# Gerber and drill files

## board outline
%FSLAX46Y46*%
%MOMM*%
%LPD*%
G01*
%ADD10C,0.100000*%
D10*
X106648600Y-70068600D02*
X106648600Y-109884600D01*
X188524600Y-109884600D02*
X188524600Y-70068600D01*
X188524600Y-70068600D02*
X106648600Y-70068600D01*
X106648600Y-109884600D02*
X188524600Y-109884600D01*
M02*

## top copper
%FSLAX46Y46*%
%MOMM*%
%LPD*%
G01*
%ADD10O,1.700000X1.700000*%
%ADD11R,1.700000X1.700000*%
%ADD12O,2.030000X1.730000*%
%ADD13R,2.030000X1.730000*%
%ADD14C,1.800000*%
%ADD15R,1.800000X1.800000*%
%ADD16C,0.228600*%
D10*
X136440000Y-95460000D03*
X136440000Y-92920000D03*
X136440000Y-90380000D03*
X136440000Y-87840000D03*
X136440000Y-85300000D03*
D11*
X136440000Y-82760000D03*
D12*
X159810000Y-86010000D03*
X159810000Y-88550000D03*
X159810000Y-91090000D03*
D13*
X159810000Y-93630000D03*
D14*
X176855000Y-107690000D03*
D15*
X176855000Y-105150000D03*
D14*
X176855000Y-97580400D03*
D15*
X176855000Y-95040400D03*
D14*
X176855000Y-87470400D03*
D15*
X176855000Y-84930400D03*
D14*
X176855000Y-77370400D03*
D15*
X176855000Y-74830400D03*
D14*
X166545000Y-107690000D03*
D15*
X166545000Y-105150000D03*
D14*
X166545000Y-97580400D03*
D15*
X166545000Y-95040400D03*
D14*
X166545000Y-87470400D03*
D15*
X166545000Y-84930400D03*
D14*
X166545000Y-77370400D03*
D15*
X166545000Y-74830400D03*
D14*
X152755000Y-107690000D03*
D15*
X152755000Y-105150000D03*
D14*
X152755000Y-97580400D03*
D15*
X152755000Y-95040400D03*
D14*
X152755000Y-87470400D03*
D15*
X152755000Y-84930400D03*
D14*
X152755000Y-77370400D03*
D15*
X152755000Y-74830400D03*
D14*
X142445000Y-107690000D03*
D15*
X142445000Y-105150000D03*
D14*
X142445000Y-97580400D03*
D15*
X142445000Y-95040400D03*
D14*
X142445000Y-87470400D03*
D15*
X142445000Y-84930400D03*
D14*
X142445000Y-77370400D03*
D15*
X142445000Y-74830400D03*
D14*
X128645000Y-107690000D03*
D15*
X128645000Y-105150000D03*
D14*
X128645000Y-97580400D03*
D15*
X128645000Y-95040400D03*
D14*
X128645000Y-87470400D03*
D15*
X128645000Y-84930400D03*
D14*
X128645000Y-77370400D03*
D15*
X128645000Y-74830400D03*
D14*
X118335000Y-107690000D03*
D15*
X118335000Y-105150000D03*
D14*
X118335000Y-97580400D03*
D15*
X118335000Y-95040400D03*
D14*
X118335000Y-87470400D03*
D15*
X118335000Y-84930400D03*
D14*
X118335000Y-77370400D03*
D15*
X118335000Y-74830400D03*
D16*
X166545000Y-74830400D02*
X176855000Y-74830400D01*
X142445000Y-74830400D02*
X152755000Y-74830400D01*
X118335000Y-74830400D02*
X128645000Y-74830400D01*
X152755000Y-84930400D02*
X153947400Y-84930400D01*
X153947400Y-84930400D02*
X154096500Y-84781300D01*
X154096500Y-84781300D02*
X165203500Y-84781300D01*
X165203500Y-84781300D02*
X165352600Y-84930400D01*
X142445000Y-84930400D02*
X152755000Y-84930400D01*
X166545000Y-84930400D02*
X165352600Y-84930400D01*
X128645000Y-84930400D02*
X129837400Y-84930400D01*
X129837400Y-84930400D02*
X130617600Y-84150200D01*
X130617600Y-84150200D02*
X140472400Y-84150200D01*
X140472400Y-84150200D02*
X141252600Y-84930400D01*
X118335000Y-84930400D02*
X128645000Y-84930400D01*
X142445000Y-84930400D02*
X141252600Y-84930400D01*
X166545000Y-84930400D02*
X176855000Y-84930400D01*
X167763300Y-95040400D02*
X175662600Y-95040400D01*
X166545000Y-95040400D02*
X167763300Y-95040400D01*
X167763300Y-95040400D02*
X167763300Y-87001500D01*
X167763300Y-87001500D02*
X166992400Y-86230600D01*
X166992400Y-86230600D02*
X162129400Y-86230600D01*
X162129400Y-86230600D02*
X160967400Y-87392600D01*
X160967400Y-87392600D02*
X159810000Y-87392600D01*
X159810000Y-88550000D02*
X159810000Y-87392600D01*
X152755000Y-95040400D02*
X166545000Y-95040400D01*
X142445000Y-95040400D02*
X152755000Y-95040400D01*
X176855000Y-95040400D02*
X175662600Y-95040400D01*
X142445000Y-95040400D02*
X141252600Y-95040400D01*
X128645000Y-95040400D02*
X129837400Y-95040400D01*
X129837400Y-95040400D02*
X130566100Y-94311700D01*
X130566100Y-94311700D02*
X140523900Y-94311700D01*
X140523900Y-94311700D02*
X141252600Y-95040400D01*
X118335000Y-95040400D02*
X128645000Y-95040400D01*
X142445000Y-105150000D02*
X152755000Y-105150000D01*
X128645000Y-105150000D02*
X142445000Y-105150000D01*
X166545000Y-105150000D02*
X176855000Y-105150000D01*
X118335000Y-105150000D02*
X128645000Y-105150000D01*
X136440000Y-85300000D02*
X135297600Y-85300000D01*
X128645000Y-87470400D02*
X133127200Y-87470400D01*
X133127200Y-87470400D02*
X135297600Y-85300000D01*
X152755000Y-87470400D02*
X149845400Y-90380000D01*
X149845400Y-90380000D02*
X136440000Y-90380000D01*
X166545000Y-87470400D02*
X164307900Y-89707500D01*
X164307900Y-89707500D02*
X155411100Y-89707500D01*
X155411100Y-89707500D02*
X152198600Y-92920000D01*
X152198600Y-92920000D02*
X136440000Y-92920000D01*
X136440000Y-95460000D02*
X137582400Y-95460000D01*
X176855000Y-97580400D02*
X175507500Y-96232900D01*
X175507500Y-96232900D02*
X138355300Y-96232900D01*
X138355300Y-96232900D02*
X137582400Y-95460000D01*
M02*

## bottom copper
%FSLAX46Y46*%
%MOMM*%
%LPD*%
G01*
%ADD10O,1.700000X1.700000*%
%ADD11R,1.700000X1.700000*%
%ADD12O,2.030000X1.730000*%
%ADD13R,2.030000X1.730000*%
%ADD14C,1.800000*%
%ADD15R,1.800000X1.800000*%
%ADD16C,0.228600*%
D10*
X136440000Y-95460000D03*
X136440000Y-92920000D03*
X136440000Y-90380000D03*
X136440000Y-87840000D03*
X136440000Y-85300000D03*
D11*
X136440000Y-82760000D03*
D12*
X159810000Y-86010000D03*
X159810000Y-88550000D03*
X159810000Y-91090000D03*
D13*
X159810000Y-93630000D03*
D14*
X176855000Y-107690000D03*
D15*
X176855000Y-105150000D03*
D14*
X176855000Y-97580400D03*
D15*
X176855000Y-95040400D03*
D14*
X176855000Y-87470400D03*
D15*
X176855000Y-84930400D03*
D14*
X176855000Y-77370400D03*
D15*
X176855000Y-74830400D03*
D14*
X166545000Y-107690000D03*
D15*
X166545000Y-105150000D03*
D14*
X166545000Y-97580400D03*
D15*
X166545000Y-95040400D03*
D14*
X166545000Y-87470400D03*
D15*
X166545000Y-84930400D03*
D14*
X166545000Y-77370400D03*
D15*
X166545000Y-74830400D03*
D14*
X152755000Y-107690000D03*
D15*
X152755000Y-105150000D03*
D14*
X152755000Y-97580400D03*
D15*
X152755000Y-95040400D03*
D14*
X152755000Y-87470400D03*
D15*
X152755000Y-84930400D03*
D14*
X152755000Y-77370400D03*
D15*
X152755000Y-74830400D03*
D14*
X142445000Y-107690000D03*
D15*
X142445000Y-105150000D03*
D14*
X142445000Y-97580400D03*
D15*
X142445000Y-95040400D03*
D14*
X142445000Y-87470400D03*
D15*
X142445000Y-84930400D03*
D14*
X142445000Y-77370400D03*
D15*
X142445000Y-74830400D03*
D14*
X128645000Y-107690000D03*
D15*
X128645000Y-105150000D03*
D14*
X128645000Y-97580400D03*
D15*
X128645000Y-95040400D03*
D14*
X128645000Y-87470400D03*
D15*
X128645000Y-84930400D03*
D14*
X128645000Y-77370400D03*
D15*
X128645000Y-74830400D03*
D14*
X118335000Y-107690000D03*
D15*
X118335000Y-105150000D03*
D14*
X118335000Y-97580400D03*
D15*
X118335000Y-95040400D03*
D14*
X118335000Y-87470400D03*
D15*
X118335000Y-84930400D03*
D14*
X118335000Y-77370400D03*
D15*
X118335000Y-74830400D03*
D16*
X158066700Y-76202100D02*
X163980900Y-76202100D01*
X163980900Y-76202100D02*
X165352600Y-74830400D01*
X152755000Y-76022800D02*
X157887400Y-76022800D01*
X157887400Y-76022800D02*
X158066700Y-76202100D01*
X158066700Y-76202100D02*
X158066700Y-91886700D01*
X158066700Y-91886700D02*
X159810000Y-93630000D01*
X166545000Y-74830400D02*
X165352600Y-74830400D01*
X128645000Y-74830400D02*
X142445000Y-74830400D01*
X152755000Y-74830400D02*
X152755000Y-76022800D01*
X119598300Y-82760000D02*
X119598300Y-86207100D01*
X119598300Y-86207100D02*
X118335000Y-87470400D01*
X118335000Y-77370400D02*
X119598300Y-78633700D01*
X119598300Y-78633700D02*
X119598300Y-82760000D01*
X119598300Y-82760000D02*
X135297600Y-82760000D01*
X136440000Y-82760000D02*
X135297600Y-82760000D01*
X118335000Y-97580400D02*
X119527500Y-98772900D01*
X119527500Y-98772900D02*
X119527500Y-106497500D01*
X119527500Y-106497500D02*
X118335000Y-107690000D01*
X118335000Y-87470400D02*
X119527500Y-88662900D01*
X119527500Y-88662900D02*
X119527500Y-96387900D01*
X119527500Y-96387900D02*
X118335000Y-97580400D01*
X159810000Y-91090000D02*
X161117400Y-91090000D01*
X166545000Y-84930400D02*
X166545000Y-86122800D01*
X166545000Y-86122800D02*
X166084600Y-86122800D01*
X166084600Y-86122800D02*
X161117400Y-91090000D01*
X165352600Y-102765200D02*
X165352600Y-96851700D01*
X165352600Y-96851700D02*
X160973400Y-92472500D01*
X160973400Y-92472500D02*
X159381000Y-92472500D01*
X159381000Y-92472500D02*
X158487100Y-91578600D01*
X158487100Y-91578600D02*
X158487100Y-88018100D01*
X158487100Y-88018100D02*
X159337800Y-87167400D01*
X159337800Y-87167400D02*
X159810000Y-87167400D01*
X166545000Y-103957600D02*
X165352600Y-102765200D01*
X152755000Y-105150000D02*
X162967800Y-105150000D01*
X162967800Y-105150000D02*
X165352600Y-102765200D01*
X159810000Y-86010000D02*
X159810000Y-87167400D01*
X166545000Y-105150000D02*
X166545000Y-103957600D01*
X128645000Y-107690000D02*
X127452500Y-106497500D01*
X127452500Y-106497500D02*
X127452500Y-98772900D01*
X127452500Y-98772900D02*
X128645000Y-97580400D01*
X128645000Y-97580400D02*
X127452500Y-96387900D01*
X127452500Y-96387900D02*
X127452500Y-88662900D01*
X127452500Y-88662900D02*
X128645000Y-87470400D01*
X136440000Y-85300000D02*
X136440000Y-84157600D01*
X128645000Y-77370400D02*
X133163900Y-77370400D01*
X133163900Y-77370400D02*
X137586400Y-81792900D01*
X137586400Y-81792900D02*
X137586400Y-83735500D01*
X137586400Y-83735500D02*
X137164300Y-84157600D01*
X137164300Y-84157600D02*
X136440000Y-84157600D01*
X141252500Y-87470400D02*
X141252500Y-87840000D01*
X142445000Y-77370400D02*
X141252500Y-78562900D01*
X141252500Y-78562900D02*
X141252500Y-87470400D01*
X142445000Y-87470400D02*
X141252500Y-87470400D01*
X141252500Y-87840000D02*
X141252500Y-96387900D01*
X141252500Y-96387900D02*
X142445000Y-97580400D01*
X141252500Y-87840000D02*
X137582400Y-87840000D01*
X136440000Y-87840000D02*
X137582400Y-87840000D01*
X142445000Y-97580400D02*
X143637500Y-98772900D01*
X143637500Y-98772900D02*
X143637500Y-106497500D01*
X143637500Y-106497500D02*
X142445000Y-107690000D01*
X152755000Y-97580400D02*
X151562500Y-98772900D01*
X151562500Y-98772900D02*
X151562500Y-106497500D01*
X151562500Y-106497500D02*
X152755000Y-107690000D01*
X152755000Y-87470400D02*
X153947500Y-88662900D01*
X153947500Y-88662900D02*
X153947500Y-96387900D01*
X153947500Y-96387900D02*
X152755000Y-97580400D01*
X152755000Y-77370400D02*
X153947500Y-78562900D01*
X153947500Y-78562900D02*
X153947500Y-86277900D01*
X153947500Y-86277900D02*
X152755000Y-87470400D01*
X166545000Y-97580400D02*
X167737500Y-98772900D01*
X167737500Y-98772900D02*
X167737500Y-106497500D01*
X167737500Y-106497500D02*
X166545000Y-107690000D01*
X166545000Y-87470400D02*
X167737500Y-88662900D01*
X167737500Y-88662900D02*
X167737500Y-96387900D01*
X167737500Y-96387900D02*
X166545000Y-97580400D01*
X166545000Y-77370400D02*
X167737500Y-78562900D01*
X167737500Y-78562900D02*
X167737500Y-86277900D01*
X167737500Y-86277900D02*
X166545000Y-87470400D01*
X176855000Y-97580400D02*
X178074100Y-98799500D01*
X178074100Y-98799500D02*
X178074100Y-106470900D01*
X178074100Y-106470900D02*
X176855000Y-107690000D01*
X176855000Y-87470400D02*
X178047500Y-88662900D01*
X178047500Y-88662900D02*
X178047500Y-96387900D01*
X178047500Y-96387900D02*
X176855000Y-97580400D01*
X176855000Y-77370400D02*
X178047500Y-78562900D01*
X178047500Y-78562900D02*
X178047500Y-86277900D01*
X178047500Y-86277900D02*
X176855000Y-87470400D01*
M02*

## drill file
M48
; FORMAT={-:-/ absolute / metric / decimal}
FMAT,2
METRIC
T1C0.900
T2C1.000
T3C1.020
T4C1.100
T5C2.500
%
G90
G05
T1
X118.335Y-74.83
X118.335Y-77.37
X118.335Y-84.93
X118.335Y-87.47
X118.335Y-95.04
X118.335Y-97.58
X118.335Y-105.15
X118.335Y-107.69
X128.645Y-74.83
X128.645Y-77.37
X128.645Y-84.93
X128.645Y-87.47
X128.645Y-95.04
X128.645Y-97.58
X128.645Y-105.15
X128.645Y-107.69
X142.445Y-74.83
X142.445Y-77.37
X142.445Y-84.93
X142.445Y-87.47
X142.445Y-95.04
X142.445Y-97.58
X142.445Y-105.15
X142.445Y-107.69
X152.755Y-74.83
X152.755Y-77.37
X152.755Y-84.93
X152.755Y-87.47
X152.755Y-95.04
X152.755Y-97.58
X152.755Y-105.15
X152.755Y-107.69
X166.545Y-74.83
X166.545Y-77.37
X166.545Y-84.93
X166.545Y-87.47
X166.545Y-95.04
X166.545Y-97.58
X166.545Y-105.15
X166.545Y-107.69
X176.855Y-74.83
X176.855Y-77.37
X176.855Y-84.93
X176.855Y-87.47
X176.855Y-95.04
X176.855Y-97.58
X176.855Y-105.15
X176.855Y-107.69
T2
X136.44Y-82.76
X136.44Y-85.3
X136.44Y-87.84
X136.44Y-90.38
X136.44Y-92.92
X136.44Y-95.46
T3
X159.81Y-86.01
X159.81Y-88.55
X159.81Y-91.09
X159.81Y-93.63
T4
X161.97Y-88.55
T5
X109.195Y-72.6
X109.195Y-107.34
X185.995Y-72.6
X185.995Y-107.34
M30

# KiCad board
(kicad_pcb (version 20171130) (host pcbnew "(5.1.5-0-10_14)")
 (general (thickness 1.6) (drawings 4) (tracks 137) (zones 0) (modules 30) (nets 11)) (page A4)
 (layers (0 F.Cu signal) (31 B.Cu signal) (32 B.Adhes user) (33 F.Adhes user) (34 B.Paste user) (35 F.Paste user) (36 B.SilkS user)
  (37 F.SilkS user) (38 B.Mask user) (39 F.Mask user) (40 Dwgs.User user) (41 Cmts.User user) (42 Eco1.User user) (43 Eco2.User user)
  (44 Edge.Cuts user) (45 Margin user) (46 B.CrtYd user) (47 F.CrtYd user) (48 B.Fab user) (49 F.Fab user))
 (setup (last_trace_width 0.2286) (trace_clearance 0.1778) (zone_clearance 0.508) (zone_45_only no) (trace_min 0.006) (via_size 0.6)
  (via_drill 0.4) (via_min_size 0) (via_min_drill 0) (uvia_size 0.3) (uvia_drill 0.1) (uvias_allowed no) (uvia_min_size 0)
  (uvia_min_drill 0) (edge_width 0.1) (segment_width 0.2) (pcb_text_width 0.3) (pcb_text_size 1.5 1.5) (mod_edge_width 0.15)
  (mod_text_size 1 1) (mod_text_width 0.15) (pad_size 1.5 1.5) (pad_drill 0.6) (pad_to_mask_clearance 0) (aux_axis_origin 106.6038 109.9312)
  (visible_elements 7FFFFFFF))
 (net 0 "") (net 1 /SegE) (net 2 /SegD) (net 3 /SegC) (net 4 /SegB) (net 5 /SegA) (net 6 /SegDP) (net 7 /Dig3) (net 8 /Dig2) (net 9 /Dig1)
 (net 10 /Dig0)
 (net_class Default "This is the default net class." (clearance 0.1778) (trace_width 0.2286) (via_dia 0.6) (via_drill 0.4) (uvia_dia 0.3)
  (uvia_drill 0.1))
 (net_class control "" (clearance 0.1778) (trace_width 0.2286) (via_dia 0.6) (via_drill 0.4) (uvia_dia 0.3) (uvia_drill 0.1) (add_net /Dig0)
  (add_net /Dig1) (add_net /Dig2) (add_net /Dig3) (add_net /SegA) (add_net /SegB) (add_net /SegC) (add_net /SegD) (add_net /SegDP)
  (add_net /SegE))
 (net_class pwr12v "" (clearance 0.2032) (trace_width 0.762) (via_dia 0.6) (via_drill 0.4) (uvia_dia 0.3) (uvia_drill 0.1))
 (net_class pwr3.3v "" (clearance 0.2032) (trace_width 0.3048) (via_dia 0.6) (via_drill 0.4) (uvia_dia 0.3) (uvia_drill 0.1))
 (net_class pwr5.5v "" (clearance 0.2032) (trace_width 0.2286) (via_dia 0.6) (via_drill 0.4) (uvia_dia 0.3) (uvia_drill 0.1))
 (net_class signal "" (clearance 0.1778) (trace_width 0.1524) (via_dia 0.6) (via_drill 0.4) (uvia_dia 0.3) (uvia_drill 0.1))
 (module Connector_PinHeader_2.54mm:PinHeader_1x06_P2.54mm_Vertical (layer F.Cu) (at 136.44 82.76)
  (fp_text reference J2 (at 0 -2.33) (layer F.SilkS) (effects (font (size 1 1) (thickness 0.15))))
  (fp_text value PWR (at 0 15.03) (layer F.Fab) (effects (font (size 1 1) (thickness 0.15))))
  (pad 6 thru_hole oval (at 0 12.7) (size 1.7 1.7) (drill 1) (layers *.Cu *.Mask) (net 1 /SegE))
  (pad 5 thru_hole oval (at 0 10.16) (size 1.7 1.7) (drill 1) (layers *.Cu *.Mask) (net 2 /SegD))
  (pad 4 thru_hole oval (at 0 7.62) (size 1.7 1.7) (drill 1) (layers *.Cu *.Mask) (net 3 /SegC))
  (pad 3 thru_hole oval (at 0 5.08) (size 1.7 1.7) (drill 1) (layers *.Cu *.Mask) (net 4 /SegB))
  (pad 2 thru_hole oval (at 0 2.54) (size 1.7 1.7) (drill 1) (layers *.Cu *.Mask) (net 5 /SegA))
  (pad 1 thru_hole rect (at 0 0) (size 1.7 1.7) (drill 1) (layers *.Cu *.Mask) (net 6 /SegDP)))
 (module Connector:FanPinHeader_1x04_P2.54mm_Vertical (layer B.Cu) (at 159.81 93.63 90)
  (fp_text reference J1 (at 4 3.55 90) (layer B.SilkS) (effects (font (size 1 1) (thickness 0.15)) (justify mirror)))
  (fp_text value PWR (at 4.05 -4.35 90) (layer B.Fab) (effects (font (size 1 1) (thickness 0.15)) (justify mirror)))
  (pad "" np_thru_hole circle (at 5.08 2.16) (size 1.1 1.1) (drill 1.1) (layers *.Cu *.Mask))
  (pad 4 thru_hole oval (at 7.62 0) (size 2.03 1.73) (drill 1.02) (layers *.Cu *.Mask) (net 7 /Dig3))
  (pad 3 thru_hole oval (at 5.08 0) (size 2.03 1.73) (drill 1.02) (layers *.Cu *.Mask) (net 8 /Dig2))
  (pad 2 thru_hole oval (at 2.54 0) (size 2.03 1.73) (drill 1.02) (layers *.Cu *.Mask) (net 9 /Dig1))
  (pad 1 thru_hole rect (at 0 0) (size 2.03 1.73) (drill 1.02) (layers *.Cu *.Mask) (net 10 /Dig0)))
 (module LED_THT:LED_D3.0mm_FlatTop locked (layer F.Cu) (at 176.855 105.15 270)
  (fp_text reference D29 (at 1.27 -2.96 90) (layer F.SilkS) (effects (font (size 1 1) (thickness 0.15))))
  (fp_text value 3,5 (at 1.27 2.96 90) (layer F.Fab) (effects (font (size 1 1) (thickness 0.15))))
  (pad 2 thru_hole circle (at 2.54 0 270) (size 1.8 1.8) (drill 0.9) (layers *.Cu *.Mask) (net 1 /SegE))
  (pad 1 thru_hole rect (at 0 0 270) (size 1.8 1.8) (drill 0.9) (layers *.Cu *.Mask) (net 7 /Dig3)))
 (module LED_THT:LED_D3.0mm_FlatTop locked (layer F.Cu) (at 176.855 95.0404 270)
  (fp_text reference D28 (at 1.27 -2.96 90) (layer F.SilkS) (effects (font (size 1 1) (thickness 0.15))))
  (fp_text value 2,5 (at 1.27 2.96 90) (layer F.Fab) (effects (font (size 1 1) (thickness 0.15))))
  (pad 2 thru_hole circle (at 2.54 0 270) (size 1.8 1.8) (drill 0.9) (layers *.Cu *.Mask) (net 1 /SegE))
  (pad 1 thru_hole rect (at 0 0 270) (size 1.8 1.8) (drill 0.9) (layers *.Cu *.Mask) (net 8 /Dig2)))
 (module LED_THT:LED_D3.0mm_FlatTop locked (layer F.Cu) (at 176.855 84.9304 270)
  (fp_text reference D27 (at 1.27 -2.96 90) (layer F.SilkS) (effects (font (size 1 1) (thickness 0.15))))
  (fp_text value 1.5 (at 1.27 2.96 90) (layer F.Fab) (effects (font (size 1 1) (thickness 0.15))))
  (pad 2 thru_hole circle (at 2.54 0 270) (size 1.8 1.8) (drill 0.9) (layers *.Cu *.Mask) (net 1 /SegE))
  (pad 1 thru_hole rect (at 0 0 270) (size 1.8 1.8) (drill 0.9) (layers *.Cu *.Mask) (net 9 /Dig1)))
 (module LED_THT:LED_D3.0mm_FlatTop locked (layer F.Cu) (at 176.855 74.8304 270)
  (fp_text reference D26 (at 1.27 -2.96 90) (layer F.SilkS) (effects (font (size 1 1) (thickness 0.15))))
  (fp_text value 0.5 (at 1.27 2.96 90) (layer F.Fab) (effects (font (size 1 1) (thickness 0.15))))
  (pad 2 thru_hole circle (at 2.54 0 270) (size 1.8 1.8) (drill 0.9) (layers *.Cu *.Mask) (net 1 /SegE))
  (pad 1 thru_hole rect (at 0 0 270) (size 1.8 1.8) (drill 0.9) (layers *.Cu *.Mask) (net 10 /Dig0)))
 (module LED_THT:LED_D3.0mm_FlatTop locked (layer F.Cu) (at 166.545 105.15 270)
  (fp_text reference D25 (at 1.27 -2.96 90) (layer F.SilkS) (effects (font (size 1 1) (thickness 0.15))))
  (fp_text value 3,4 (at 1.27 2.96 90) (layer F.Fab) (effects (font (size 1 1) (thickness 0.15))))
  (pad 2 thru_hole circle (at 2.54 0 270) (size 1.8 1.8) (drill 0.9) (layers *.Cu *.Mask) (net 2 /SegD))
  (pad 1 thru_hole rect (at 0 0 270) (size 1.8 1.8) (drill 0.9) (layers *.Cu *.Mask) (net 7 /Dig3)))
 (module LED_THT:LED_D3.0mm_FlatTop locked (layer F.Cu) (at 166.545 95.0404 270)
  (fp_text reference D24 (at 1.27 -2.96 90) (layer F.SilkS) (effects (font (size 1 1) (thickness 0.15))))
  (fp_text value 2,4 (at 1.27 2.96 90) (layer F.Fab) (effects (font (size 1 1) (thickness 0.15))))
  (pad 2 thru_hole circle (at 2.54 0 270) (size 1.8 1.8) (drill 0.9) (layers *.Cu *.Mask) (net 2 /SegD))
  (pad 1 thru_hole rect (at 0 0 270) (size 1.8 1.8) (drill 0.9) (layers *.Cu *.Mask) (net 8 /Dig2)))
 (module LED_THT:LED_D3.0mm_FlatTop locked (layer F.Cu) (at 166.545 84.9304 270)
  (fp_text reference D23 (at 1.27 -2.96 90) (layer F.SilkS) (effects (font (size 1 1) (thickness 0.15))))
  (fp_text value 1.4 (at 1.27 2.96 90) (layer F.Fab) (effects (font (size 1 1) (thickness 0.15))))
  (pad 2 thru_hole circle (at 2.54 0 270) (size 1.8 1.8) (drill 0.9) (layers *.Cu *.Mask) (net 2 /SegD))
  (pad 1 thru_hole rect (at 0 0 270) (size 1.8 1.8) (drill 0.9) (layers *.Cu *.Mask) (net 9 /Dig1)))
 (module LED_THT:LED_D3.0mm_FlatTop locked (layer F.Cu) (at 166.545 74.8304 270)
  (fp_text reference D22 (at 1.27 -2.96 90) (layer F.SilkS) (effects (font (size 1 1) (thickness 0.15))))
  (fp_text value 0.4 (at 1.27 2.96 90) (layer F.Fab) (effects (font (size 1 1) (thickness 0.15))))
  (pad 2 thru_hole circle (at 2.54 0 270) (size 1.8 1.8) (drill 0.9) (layers *.Cu *.Mask) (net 2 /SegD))
  (pad 1 thru_hole rect (at 0 0 270) (size 1.8 1.8) (drill 0.9) (layers *.Cu *.Mask) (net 10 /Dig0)))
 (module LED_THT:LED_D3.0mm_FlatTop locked (layer F.Cu) (at 152.755 105.15 270)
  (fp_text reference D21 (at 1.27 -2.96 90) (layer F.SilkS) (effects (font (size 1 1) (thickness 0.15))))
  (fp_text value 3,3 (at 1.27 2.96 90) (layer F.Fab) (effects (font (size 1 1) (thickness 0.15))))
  (pad 2 thru_hole circle (at 2.54 0 270) (size 1.8 1.8) (drill 0.9) (layers *.Cu *.Mask) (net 3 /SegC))
  (pad 1 thru_hole rect (at 0 0 270) (size 1.8 1.8) (drill 0.9) (layers *.Cu *.Mask) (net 7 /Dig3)))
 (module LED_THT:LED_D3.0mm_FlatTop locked (layer F.Cu) (at 152.755 95.0404 270)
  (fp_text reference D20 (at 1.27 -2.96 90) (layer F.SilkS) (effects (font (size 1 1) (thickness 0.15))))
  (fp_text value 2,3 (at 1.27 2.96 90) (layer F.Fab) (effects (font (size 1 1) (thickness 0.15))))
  (pad 2 thru_hole circle (at 2.54 0 270) (size 1.8 1.8) (drill 0.9) (layers *.Cu *.Mask) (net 3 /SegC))
  (pad 1 thru_hole rect (at 0 0 270) (size 1.8 1.8) (drill 0.9) (layers *.Cu *.Mask) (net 8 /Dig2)))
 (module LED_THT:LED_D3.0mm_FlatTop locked (layer F.Cu) (at 152.755 84.9304 270)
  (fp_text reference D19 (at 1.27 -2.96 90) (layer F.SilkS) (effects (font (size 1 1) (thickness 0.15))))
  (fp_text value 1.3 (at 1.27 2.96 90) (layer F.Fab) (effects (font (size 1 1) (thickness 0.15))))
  (pad 2 thru_hole circle (at 2.54 0 270) (size 1.8 1.8) (drill 0.9) (layers *.Cu *.Mask) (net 3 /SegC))
  (pad 1 thru_hole rect (at 0 0 270) (size 1.8 1.8) (drill 0.9) (layers *.Cu *.Mask) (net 9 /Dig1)))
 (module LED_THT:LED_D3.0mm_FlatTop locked (layer F.Cu) (at 152.755 74.8304 270)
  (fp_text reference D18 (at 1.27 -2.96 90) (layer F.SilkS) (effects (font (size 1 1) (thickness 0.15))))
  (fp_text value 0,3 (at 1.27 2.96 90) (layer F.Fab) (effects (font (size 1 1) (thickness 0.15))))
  (pad 2 thru_hole circle (at 2.54 0 270) (size 1.8 1.8) (drill 0.9) (layers *.Cu *.Mask) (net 3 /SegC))
  (pad 1 thru_hole rect (at 0 0 270) (size 1.8 1.8) (drill 0.9) (layers *.Cu *.Mask) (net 10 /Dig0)))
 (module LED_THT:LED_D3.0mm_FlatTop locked (layer F.Cu) (at 142.445 105.15 270)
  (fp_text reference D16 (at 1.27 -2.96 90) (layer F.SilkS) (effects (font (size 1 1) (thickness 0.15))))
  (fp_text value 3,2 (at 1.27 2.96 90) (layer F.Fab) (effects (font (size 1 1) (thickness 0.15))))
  (pad 2 thru_hole circle (at 2.54 0 270) (size 1.8 1.8) (drill 0.9) (layers *.Cu *.Mask) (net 4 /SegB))
  (pad 1 thru_hole rect (at 0 0 270) (size 1.8 1.8) (drill 0.9) (layers *.Cu *.Mask) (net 7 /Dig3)))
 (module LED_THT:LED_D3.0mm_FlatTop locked (layer F.Cu) (at 142.445 95.0404 270)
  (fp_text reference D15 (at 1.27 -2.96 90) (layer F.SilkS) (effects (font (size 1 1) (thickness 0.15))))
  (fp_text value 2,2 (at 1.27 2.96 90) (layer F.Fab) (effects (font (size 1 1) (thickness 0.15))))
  (pad 2 thru_hole circle (at 2.54 0 270) (size 1.8 1.8) (drill 0.9) (layers *.Cu *.Mask) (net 4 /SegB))
  (pad 1 thru_hole rect (at 0 0 270) (size 1.8 1.8) (drill 0.9) (layers *.Cu *.Mask) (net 8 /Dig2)))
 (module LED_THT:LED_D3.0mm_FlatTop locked (layer F.Cu) (at 142.445 84.9304 270)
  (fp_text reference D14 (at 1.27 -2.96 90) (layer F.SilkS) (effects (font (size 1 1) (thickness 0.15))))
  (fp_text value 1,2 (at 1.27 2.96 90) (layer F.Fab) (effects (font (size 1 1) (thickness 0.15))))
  (pad 2 thru_hole circle (at 2.54 0 270) (size 1.8 1.8) (drill 0.9) (layers *.Cu *.Mask) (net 4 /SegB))
  (pad 1 thru_hole rect (at 0 0 270) (size 1.8 1.8) (drill 0.9) (layers *.Cu *.Mask) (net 9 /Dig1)))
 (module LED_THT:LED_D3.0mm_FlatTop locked (layer F.Cu) (at 142.445 74.8304 270)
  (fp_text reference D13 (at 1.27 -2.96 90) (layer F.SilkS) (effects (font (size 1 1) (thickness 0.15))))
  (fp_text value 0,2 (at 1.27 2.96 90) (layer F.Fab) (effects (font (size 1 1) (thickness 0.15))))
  (pad 2 thru_hole circle (at 2.54 0 270) (size 1.8 1.8) (drill 0.9) (layers *.Cu *.Mask) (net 4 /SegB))
  (pad 1 thru_hole rect (at 0 0 270) (size 1.8 1.8) (drill 0.9) (layers *.Cu *.Mask) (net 10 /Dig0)))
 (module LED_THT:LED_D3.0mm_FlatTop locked (layer F.Cu) (at 128.645 105.15 270)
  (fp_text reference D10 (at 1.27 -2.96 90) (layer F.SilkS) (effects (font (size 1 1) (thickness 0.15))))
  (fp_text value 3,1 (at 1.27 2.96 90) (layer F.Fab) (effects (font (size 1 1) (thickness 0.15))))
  (pad 2 thru_hole circle (at 2.54 0 270) (size 1.8 1.8) (drill 0.9) (layers *.Cu *.Mask) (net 5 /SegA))
  (pad 1 thru_hole rect (at 0 0 270) (size 1.8 1.8) (drill 0.9) (layers *.Cu *.Mask) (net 7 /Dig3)))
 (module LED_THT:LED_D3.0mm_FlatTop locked (layer F.Cu) (at 128.645 95.0404 270)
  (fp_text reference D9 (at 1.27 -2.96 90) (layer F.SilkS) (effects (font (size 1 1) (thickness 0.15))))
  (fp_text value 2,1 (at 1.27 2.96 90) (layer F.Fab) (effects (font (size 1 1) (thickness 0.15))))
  (pad 2 thru_hole circle (at 2.54 0 270) (size 1.8 1.8) (drill 0.9) (layers *.Cu *.Mask) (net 5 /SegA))
  (pad 1 thru_hole rect (at 0 0 270) (size 1.8 1.8) (drill 0.9) (layers *.Cu *.Mask) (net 8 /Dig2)))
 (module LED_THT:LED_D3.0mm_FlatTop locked (layer F.Cu) (at 128.645 84.9304 270)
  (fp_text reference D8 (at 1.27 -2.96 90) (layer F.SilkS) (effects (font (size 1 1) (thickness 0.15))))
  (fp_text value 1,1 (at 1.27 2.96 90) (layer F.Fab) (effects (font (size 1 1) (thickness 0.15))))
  (pad 2 thru_hole circle (at 2.54 0 270) (size 1.8 1.8) (drill 0.9) (layers *.Cu *.Mask) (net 5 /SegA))
  (pad 1 thru_hole rect (at 0 0 270) (size 1.8 1.8) (drill 0.9) (layers *.Cu *.Mask) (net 9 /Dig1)))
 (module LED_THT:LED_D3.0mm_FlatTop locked (layer F.Cu) (at 128.645 74.8304 270)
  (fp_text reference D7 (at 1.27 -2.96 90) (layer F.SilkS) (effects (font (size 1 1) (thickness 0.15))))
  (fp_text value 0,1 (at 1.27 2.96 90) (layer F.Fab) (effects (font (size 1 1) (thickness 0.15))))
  (pad 2 thru_hole circle (at 2.54 0 270) (size 1.8 1.8) (drill 0.9) (layers *.Cu *.Mask) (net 5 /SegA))
  (pad 1 thru_hole rect (at 0 0 270) (size 1.8 1.8) (drill 0.9) (layers *.Cu *.Mask) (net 10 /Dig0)))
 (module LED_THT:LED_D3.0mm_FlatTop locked (layer F.Cu) (at 118.335 105.15 270)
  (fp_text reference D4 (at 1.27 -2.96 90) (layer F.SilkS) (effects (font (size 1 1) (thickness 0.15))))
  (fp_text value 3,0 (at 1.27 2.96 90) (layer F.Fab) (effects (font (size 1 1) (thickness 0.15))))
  (pad 2 thru_hole circle (at 2.54 0 270) (size 1.8 1.8) (drill 0.9) (layers *.Cu *.Mask) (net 6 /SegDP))
  (pad 1 thru_hole rect (at 0 0 270) (size 1.8 1.8) (drill 0.9) (layers *.Cu *.Mask) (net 7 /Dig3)))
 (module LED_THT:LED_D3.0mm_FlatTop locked (layer F.Cu) (at 118.335 95.0404 270)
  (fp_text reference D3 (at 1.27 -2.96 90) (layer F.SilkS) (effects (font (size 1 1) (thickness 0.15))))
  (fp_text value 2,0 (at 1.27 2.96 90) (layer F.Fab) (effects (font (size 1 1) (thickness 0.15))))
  (pad 2 thru_hole circle (at 2.54 0 270) (size 1.8 1.8) (drill 0.9) (layers *.Cu *.Mask) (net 6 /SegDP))
  (pad 1 thru_hole rect (at 0 0 270) (size 1.8 1.8) (drill 0.9) (layers *.Cu *.Mask) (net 8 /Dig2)))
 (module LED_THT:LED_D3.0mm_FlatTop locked (layer F.Cu) (at 118.335 84.9304 270)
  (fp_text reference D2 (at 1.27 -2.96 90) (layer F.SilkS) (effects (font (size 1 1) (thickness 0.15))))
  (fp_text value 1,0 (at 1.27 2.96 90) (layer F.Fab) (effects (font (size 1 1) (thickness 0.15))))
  (pad 2 thru_hole circle (at 2.54 0 270) (size 1.8 1.8) (drill 0.9) (layers *.Cu *.Mask) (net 6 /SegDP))
  (pad 1 thru_hole rect (at 0 0 270) (size 1.8 1.8) (drill 0.9) (layers *.Cu *.Mask) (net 9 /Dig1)))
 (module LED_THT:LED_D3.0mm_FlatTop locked (layer F.Cu) (at 118.335 74.8304 270)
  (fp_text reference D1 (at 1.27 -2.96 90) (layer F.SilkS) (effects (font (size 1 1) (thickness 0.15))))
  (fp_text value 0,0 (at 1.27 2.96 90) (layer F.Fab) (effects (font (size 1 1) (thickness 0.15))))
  (pad 2 thru_hole circle (at 2.54 0 270) (size 1.8 1.8) (drill 0.9) (layers *.Cu *.Mask) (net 6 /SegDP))
  (pad 1 thru_hole rect (at 0 0 270) (size 1.8 1.8) (drill 0.9) (layers *.Cu *.Mask) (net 10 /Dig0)))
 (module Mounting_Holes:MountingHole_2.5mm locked (layer F.Cu) (at 109.195 72.6004)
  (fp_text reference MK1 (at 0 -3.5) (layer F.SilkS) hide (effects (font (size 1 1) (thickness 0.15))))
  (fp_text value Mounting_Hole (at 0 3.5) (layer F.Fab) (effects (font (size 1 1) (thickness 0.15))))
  (pad 1 np_thru_hole circle (at 0 0) (size 2.5 2.5) (drill 2.5) (layers *.Cu *.Mask)))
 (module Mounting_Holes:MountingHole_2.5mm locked (layer F.Cu) (at 185.995 72.6004)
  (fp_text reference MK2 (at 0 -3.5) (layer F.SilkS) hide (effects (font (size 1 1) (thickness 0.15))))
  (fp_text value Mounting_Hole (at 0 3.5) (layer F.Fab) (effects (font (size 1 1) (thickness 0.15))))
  (pad 1 np_thru_hole circle (at 0 0) (size 2.5 2.5) (drill 2.5) (layers *.Cu *.Mask)))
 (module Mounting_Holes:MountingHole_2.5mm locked (layer F.Cu) (at 109.195 107.34)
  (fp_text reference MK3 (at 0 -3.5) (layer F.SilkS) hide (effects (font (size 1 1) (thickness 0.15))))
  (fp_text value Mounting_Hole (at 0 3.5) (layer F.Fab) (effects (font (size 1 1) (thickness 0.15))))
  (pad 1 np_thru_hole circle (at 0 0) (size 2.5 2.5) (drill 2.5) (layers *.Cu *.Mask)))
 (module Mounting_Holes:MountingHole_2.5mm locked (layer F.Cu) (at 185.995 107.34)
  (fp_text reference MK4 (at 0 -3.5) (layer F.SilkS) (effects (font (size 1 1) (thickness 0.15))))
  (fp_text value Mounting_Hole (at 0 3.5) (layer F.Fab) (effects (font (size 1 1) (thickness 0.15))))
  (pad 1 np_thru_hole circle (at 0 0) (size 2.5 2.5) (drill 2.5) (layers *.Cu *.Mask)))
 (gr_line (start 106.6486 70.0686) (end 106.6486 109.8846) (layer Edge.Cuts) (width 0.1))
 (gr_line (start 188.5246 109.8846) (end 188.5246 70.0686) (layer Edge.Cuts) (width 0.1))
 (gr_line (start 188.5246 70.0686) (end 106.6486 70.0686) (layer Edge.Cuts) (width 0.1))
 (gr_line (start 106.6486 109.8846) (end 188.5246 109.8846) (layer Edge.Cuts) (width 0.1))
 (segment (start 158.0667 76.2021) (end 163.9809 76.2021) (width 0.2286) (layer B.Cu) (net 10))
 (segment (start 163.9809 76.2021) (end 165.3526 74.8304) (width 0.2286) (layer B.Cu) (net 10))
 (segment (start 152.755 76.0228) (end 157.8874 76.0228) (width 0.2286) (layer B.Cu) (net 10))
 (segment (start 157.8874 76.0228) (end 158.0667 76.2021) (width 0.2286) (layer B.Cu) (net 10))
 (segment (start 158.0667 76.2021) (end 158.0667 91.8867) (width 0.2286) (layer B.Cu) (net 10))
 (segment (start 158.0667 91.8867) (end 159.81 93.63) (width 0.2286) (layer B.Cu) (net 10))
 (segment (start 166.545 74.8304) (end 165.3526 74.8304) (width 0.2286) (layer B.Cu) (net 10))
 (segment (start 128.645 74.8304) (end 142.445 74.8304) (width 0.2286) (layer B.Cu) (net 10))
 (segment (start 152.755 74.8304) (end 152.755 76.0228) (width 0.2286) (layer B.Cu) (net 10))
 (segment (start 166.545 74.8304) (end 176.855 74.8304) (width 0.2286) (layer F.Cu) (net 10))
 (segment (start 142.445 74.8304) (end 152.755 74.8304) (width 0.2286) (layer F.Cu) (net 10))
 (segment (start 118.335 74.8304) (end 128.645 74.8304) (width 0.2286) (layer F.Cu) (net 10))
 (segment (start 119.5983 82.76) (end 119.5983 86.2071) (width 0.2286) (layer B.Cu) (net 6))
 (segment (start 119.5983 86.2071) (end 118.335 87.4704) (width 0.2286) (layer B.Cu) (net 6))
 (segment (start 118.335 77.3704) (end 119.5983 78.6337) (width 0.2286) (layer B.Cu) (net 6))
 (segment (start 119.5983 78.6337) (end 119.5983 82.76) (width 0.2286) (layer B.Cu) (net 6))
 (segment (start 119.5983 82.76) (end 135.2976 82.76) (width 0.2286) (layer B.Cu) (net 6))
 (segment (start 136.44 82.76) (end 135.2976 82.76) (width 0.2286) (layer B.Cu) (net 6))
 (segment (start 118.335 97.5804) (end 119.5275 98.7729) (width 0.2286) (layer B.Cu) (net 6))
 (segment (start 119.5275 98.7729) (end 119.5275 106.4975) (width 0.2286) (layer B.Cu) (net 6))
 (segment (start 119.5275 106.4975) (end 118.335 107.69) (width 0.2286) (layer B.Cu) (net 6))
 (segment (start 118.335 87.4704) (end 119.5275 88.6629) (width 0.2286) (layer B.Cu) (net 6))
 (segment (start 119.5275 88.6629) (end 119.5275 96.3879) (width 0.2286) (layer B.Cu) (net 6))
 (segment (start 119.5275 96.3879) (end 118.335 97.5804) (width 0.2286) (layer B.Cu) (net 6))
 (segment (start 159.81 91.09) (end 161.1174 91.09) (width 0.2286) (layer B.Cu) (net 9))
 (segment (start 166.545 84.9304) (end 166.545 86.1228) (width 0.2286) (layer B.Cu) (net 9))
 (segment (start 166.545 86.1228) (end 166.0846 86.1228) (width 0.2286) (layer B.Cu) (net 9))
 (segment (start 166.0846 86.1228) (end 161.1174 91.09) (width 0.2286) (layer B.Cu) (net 9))
 (segment (start 152.755 84.9304) (end 153.9474 84.9304) (width 0.2286) (layer F.Cu) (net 9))
 (segment (start 153.9474 84.9304) (end 154.0965 84.7813) (width 0.2286) (layer F.Cu) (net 9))
 (segment (start 154.0965 84.7813) (end 165.2035 84.7813) (width 0.2286) (layer F.Cu) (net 9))
 (segment (start 165.2035 84.7813) (end 165.3526 84.9304) (width 0.2286) (layer F.Cu) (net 9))
 (segment (start 142.445 84.9304) (end 152.755 84.9304) (width 0.2286) (layer F.Cu) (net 9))
 (segment (start 166.545 84.9304) (end 165.3526 84.9304) (width 0.2286) (layer F.Cu) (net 9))
 (segment (start 128.645 84.9304) (end 129.8374 84.9304) (width 0.2286) (layer F.Cu) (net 9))
 (segment (start 129.8374 84.9304) (end 130.6176 84.1502) (width 0.2286) (layer F.Cu) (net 9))
 (segment (start 130.6176 84.1502) (end 140.4724 84.1502) (width 0.2286) (layer F.Cu) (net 9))
 (segment (start 140.4724 84.1502) (end 141.2526 84.9304) (width 0.2286) (layer F.Cu) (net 9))
 (segment (start 118.335 84.9304) (end 128.645 84.9304) (width 0.2286) (layer F.Cu) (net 9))
 (segment (start 142.445 84.9304) (end 141.2526 84.9304) (width 0.2286) (layer F.Cu) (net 9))
 (segment (start 166.545 84.9304) (end 176.855 84.9304) (width 0.2286) (layer F.Cu) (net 9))
 (segment (start 167.7633 95.0404) (end 175.6626 95.0404) (width 0.2286) (layer F.Cu) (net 8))
 (segment (start 166.545 95.0404) (end 167.7633 95.0404) (width 0.2286) (layer F.Cu) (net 8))
 (segment (start 167.7633 95.0404) (end 167.7633 87.0015) (width 0.2286) (layer F.Cu) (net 8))
 (segment (start 167.7633 87.0015) (end 166.9924 86.2306) (width 0.2286) (layer F.Cu) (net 8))
 (segment (start 166.9924 86.2306) (end 162.1294 86.2306) (width 0.2286) (layer F.Cu) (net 8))
 (segment (start 162.1294 86.2306) (end 160.9674 87.3926) (width 0.2286) (layer F.Cu) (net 8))
 (segment (start 160.9674 87.3926) (end 159.81 87.3926) (width 0.2286) (layer F.Cu) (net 8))
 (segment (start 159.81 88.55) (end 159.81 87.3926) (width 0.2286) (layer F.Cu) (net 8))
 (segment (start 152.755 95.0404) (end 166.545 95.0404) (width 0.2286) (layer F.Cu) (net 8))
 (segment (start 142.445 95.0404) (end 152.755 95.0404) (width 0.2286) (layer F.Cu) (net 8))
 (segment (start 176.855 95.0404) (end 175.6626 95.0404) (width 0.2286) (layer F.Cu) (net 8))
 (segment (start 142.445 95.0404) (end 141.2526 95.0404) (width 0.2286) (layer F.Cu) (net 8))
 (segment (start 128.645 95.0404) (end 129.8374 95.0404) (width 0.2286) (layer F.Cu) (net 8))
 (segment (start 129.8374 95.0404) (end 130.5661 94.3117) (width 0.2286) (layer F.Cu) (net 8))
 (segment (start 130.5661 94.3117) (end 140.5239 94.3117) (width 0.2286) (layer F.Cu) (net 8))
 (segment (start 140.5239 94.3117) (end 141.2526 95.0404) (width 0.2286) (layer F.Cu) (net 8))
 (segment (start 118.335 95.0404) (end 128.645 95.0404) (width 0.2286) (layer F.Cu) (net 8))
 (segment (start 165.3526 102.7652) (end 165.3526 96.8517) (width 0.2286) (layer B.Cu) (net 7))
 (segment (start 165.3526 96.8517) (end 160.9734 92.4725) (width 0.2286) (layer B.Cu) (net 7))
 (segment (start 160.9734 92.4725) (end 159.381 92.4725) (width 0.2286) (layer B.Cu) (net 7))
 (segment (start 159.381 92.4725) (end 158.4871 91.5786) (width 0.2286) (layer B.Cu) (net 7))
 (segment (start 158.4871 91.5786) (end 158.4871 88.0181) (width 0.2286) (layer B.Cu) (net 7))
 (segment (start 158.4871 88.0181) (end 159.3378 87.1674) (width 0.2286) (layer B.Cu) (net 7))
 (segment (start 159.3378 87.1674) (end 159.81 87.1674) (width 0.2286) (layer B.Cu) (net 7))
 (segment (start 166.545 103.9576) (end 165.3526 102.7652) (width 0.2286) (layer B.Cu) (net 7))
 (segment (start 152.755 105.15) (end 162.9678 105.15) (width 0.2286) (layer B.Cu) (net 7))
 (segment (start 162.9678 105.15) (end 165.3526 102.7652) (width 0.2286) (layer B.Cu) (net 7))
 (segment (start 142.445 105.15) (end 152.755 105.15) (width 0.2286) (layer F.Cu) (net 7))
 (segment (start 128.645 105.15) (end 142.445 105.15) (width 0.2286) (layer F.Cu) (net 7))
 (segment (start 159.81 86.01) (end 159.81 87.1674) (width 0.2286) (layer B.Cu) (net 7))
 (segment (start 166.545 105.15) (end 166.545 103.9576) (width 0.2286) (layer B.Cu) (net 7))
 (segment (start 166.545 105.15) (end 176.855 105.15) (width 0.2286) (layer F.Cu) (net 7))
 (segment (start 118.335 105.15) (end 128.645 105.15) (width 0.2286) (layer F.Cu) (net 7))
 (segment (start 128.645 107.69) (end 127.4525 106.4975) (width 0.2286) (layer B.Cu) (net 5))
 (segment (start 127.4525 106.4975) (end 127.4525 98.7729) (width 0.2286) (layer B.Cu) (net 5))
 (segment (start 127.4525 98.7729) (end 128.645 97.5804) (width 0.2286) (layer B.Cu) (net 5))
 (segment (start 128.645 97.5804) (end 127.4525 96.3879) (width 0.2286) (layer B.Cu) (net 5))
 (segment (start 127.4525 96.3879) (end 127.4525 88.6629) (width 0.2286) (layer B.Cu) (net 5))
 (segment (start 127.4525 88.6629) (end 128.645 87.4704) (width 0.2286) (layer B.Cu) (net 5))
 (segment (start 136.44 85.3) (end 135.2976 85.3) (width 0.2286) (layer F.Cu) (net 5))
 (segment (start 128.645 87.4704) (end 133.1272 87.4704) (width 0.2286) (layer F.Cu) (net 5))
 (segment (start 133.1272 87.4704) (end 135.2976 85.3) (width 0.2286) (layer F.Cu) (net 5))
 (segment (start 136.44 85.3) (end 136.44 84.1576) (width 0.2286) (layer B.Cu) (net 5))
 (segment (start 128.645 77.3704) (end 133.1639 77.3704) (width 0.2286) (layer B.Cu) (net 5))
 (segment (start 133.1639 77.3704) (end 137.5864 81.7929) (width 0.2286) (layer B.Cu) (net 5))
 (segment (start 137.5864 81.7929) (end 137.5864 83.7355) (width 0.2286) (layer B.Cu) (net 5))
 (segment (start 137.5864 83.7355) (end 137.1643 84.1576) (width 0.2286) (layer B.Cu) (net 5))
 (segment (start 137.1643 84.1576) (end 136.44 84.1576) (width 0.2286) (layer B.Cu) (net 5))
 (segment (start 141.2525 87.4704) (end 141.2525 87.84) (width 0.2286) (layer B.Cu) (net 4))
 (segment (start 142.445 77.3704) (end 141.2525 78.5629) (width 0.2286) (layer B.Cu) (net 4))
 (segment (start 141.2525 78.5629) (end 141.2525 87.4704) (width 0.2286) (layer B.Cu) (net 4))
 (segment (start 142.445 87.4704) (end 141.2525 87.4704) (width 0.2286) (layer B.Cu) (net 4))
 (segment (start 141.2525 87.84) (end 141.2525 96.3879) (width 0.2286) (layer B.Cu) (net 4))
 (segment (start 141.2525 96.3879) (end 142.445 97.5804) (width 0.2286) (layer B.Cu) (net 4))
 (segment (start 141.2525 87.84) (end 137.5824 87.84) (width 0.2286) (layer B.Cu) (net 4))
 (segment (start 136.44 87.84) (end 137.5824 87.84) (width 0.2286) (layer B.Cu) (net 4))
 (segment (start 142.445 97.5804) (end 143.6375 98.7729) (width 0.2286) (layer B.Cu) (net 4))
 (segment (start 143.6375 98.7729) (end 143.6375 106.4975) (width 0.2286) (layer B.Cu) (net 4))
 (segment (start 143.6375 106.4975) (end 142.445 107.69) (width 0.2286) (layer B.Cu) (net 4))
 (segment (start 152.755 87.4704) (end 149.8454 90.38) (width 0.2286) (layer F.Cu) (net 3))
 (segment (start 149.8454 90.38) (end 136.44 90.38) (width 0.2286) (layer F.Cu) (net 3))
 (segment (start 152.755 97.5804) (end 151.5625 98.7729) (width 0.2286) (layer B.Cu) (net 3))
 (segment (start 151.5625 98.7729) (end 151.5625 106.4975) (width 0.2286) (layer B.Cu) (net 3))
 (segment (start 151.5625 106.4975) (end 152.755 107.69) (width 0.2286) (layer B.Cu) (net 3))
 (segment (start 152.755 87.4704) (end 153.9475 88.6629) (width 0.2286) (layer B.Cu) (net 3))
 (segment (start 153.9475 88.6629) (end 153.9475 96.3879) (width 0.2286) (layer B.Cu) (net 3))
 (segment (start 153.9475 96.3879) (end 152.755 97.5804) (width 0.2286) (layer B.Cu) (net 3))
 (segment (start 152.755 77.3704) (end 153.9475 78.5629) (width 0.2286) (layer B.Cu) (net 3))
 (segment (start 153.9475 78.5629) (end 153.9475 86.2779) (width 0.2286) (layer B.Cu) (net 3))
 (segment (start 153.9475 86.2779) (end 152.755 87.4704) (width 0.2286) (layer B.Cu) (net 3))
 (segment (start 166.545 87.4704) (end 164.3079 89.7075) (width 0.2286) (layer F.Cu) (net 2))
 (segment (start 164.3079 89.7075) (end 155.4111 89.7075) (width 0.2286) (layer F.Cu) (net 2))
 (segment (start 155.4111 89.7075) (end 152.1986 92.92) (width 0.2286) (layer F.Cu) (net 2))
 (segment (start 152.1986 92.92) (end 136.44 92.92) (width 0.2286) (layer F.Cu) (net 2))
 (segment (start 166.545 97.5804) (end 167.7375 98.7729) (width 0.2286) (layer B.Cu) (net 2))
 (segment (start 167.7375 98.7729) (end 167.7375 106.4975) (width 0.2286) (layer B.Cu) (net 2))
 (segment (start 167.7375 106.4975) (end 166.545 107.69) (width 0.2286) (layer B.Cu) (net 2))
 (segment (start 166.545 87.4704) (end 167.7375 88.6629) (width 0.2286) (layer B.Cu) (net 2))
 (segment (start 167.7375 88.6629) (end 167.7375 96.3879) (width 0.2286) (layer B.Cu) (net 2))
 (segment (start 167.7375 96.3879) (end 166.545 97.5804) (width 0.2286) (layer B.Cu) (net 2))
 (segment (start 166.545 77.3704) (end 167.7375 78.5629) (width 0.2286) (layer B.Cu) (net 2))
 (segment (start 167.7375 78.5629) (end 167.7375 86.2779) (width 0.2286) (layer B.Cu) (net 2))
 (segment (start 167.7375 86.2779) (end 166.545 87.4704) (width 0.2286) (layer B.Cu) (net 2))
 (segment (start 136.44 95.46) (end 137.5824 95.46) (width 0.2286) (layer F.Cu) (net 1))
 (segment (start 176.855 97.5804) (end 175.5075 96.2329) (width 0.2286) (layer F.Cu) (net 1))
 (segment (start 175.5075 96.2329) (end 138.3553 96.2329) (width 0.2286) (layer F.Cu) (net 1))
 (segment (start 138.3553 96.2329) (end 137.5824 95.46) (width 0.2286) (layer F.Cu) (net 1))
 (segment (start 176.855 97.5804) (end 178.0741 98.7995) (width 0.2286) (layer B.Cu) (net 1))
 (segment (start 178.0741 98.7995) (end 178.0741 106.4709) (width 0.2286) (layer B.Cu) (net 1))
 (segment (start 178.0741 106.4709) (end 176.855 107.69) (width 0.2286) (layer B.Cu) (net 1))
 (segment (start 176.855 87.4704) (end 178.0475 88.6629) (width 0.2286) (layer B.Cu) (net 1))
 (segment (start 178.0475 88.6629) (end 178.0475 96.3879) (width 0.2286) (layer B.Cu) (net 1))
 (segment (start 178.0475 96.3879) (end 176.855 97.5804) (width 0.2286) (layer B.Cu) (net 1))
 (segment (start 176.855 77.3704) (end 178.0475 78.5629) (width 0.2286) (layer B.Cu) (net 1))
 (segment (start 178.0475 78.5629) (end 178.0475 86.2779) (width 0.2286) (layer B.Cu) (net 1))
 (segment (start 178.0475 86.2779) (end 176.855 87.4704) (width 0.2286) (layer B.Cu) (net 1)))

